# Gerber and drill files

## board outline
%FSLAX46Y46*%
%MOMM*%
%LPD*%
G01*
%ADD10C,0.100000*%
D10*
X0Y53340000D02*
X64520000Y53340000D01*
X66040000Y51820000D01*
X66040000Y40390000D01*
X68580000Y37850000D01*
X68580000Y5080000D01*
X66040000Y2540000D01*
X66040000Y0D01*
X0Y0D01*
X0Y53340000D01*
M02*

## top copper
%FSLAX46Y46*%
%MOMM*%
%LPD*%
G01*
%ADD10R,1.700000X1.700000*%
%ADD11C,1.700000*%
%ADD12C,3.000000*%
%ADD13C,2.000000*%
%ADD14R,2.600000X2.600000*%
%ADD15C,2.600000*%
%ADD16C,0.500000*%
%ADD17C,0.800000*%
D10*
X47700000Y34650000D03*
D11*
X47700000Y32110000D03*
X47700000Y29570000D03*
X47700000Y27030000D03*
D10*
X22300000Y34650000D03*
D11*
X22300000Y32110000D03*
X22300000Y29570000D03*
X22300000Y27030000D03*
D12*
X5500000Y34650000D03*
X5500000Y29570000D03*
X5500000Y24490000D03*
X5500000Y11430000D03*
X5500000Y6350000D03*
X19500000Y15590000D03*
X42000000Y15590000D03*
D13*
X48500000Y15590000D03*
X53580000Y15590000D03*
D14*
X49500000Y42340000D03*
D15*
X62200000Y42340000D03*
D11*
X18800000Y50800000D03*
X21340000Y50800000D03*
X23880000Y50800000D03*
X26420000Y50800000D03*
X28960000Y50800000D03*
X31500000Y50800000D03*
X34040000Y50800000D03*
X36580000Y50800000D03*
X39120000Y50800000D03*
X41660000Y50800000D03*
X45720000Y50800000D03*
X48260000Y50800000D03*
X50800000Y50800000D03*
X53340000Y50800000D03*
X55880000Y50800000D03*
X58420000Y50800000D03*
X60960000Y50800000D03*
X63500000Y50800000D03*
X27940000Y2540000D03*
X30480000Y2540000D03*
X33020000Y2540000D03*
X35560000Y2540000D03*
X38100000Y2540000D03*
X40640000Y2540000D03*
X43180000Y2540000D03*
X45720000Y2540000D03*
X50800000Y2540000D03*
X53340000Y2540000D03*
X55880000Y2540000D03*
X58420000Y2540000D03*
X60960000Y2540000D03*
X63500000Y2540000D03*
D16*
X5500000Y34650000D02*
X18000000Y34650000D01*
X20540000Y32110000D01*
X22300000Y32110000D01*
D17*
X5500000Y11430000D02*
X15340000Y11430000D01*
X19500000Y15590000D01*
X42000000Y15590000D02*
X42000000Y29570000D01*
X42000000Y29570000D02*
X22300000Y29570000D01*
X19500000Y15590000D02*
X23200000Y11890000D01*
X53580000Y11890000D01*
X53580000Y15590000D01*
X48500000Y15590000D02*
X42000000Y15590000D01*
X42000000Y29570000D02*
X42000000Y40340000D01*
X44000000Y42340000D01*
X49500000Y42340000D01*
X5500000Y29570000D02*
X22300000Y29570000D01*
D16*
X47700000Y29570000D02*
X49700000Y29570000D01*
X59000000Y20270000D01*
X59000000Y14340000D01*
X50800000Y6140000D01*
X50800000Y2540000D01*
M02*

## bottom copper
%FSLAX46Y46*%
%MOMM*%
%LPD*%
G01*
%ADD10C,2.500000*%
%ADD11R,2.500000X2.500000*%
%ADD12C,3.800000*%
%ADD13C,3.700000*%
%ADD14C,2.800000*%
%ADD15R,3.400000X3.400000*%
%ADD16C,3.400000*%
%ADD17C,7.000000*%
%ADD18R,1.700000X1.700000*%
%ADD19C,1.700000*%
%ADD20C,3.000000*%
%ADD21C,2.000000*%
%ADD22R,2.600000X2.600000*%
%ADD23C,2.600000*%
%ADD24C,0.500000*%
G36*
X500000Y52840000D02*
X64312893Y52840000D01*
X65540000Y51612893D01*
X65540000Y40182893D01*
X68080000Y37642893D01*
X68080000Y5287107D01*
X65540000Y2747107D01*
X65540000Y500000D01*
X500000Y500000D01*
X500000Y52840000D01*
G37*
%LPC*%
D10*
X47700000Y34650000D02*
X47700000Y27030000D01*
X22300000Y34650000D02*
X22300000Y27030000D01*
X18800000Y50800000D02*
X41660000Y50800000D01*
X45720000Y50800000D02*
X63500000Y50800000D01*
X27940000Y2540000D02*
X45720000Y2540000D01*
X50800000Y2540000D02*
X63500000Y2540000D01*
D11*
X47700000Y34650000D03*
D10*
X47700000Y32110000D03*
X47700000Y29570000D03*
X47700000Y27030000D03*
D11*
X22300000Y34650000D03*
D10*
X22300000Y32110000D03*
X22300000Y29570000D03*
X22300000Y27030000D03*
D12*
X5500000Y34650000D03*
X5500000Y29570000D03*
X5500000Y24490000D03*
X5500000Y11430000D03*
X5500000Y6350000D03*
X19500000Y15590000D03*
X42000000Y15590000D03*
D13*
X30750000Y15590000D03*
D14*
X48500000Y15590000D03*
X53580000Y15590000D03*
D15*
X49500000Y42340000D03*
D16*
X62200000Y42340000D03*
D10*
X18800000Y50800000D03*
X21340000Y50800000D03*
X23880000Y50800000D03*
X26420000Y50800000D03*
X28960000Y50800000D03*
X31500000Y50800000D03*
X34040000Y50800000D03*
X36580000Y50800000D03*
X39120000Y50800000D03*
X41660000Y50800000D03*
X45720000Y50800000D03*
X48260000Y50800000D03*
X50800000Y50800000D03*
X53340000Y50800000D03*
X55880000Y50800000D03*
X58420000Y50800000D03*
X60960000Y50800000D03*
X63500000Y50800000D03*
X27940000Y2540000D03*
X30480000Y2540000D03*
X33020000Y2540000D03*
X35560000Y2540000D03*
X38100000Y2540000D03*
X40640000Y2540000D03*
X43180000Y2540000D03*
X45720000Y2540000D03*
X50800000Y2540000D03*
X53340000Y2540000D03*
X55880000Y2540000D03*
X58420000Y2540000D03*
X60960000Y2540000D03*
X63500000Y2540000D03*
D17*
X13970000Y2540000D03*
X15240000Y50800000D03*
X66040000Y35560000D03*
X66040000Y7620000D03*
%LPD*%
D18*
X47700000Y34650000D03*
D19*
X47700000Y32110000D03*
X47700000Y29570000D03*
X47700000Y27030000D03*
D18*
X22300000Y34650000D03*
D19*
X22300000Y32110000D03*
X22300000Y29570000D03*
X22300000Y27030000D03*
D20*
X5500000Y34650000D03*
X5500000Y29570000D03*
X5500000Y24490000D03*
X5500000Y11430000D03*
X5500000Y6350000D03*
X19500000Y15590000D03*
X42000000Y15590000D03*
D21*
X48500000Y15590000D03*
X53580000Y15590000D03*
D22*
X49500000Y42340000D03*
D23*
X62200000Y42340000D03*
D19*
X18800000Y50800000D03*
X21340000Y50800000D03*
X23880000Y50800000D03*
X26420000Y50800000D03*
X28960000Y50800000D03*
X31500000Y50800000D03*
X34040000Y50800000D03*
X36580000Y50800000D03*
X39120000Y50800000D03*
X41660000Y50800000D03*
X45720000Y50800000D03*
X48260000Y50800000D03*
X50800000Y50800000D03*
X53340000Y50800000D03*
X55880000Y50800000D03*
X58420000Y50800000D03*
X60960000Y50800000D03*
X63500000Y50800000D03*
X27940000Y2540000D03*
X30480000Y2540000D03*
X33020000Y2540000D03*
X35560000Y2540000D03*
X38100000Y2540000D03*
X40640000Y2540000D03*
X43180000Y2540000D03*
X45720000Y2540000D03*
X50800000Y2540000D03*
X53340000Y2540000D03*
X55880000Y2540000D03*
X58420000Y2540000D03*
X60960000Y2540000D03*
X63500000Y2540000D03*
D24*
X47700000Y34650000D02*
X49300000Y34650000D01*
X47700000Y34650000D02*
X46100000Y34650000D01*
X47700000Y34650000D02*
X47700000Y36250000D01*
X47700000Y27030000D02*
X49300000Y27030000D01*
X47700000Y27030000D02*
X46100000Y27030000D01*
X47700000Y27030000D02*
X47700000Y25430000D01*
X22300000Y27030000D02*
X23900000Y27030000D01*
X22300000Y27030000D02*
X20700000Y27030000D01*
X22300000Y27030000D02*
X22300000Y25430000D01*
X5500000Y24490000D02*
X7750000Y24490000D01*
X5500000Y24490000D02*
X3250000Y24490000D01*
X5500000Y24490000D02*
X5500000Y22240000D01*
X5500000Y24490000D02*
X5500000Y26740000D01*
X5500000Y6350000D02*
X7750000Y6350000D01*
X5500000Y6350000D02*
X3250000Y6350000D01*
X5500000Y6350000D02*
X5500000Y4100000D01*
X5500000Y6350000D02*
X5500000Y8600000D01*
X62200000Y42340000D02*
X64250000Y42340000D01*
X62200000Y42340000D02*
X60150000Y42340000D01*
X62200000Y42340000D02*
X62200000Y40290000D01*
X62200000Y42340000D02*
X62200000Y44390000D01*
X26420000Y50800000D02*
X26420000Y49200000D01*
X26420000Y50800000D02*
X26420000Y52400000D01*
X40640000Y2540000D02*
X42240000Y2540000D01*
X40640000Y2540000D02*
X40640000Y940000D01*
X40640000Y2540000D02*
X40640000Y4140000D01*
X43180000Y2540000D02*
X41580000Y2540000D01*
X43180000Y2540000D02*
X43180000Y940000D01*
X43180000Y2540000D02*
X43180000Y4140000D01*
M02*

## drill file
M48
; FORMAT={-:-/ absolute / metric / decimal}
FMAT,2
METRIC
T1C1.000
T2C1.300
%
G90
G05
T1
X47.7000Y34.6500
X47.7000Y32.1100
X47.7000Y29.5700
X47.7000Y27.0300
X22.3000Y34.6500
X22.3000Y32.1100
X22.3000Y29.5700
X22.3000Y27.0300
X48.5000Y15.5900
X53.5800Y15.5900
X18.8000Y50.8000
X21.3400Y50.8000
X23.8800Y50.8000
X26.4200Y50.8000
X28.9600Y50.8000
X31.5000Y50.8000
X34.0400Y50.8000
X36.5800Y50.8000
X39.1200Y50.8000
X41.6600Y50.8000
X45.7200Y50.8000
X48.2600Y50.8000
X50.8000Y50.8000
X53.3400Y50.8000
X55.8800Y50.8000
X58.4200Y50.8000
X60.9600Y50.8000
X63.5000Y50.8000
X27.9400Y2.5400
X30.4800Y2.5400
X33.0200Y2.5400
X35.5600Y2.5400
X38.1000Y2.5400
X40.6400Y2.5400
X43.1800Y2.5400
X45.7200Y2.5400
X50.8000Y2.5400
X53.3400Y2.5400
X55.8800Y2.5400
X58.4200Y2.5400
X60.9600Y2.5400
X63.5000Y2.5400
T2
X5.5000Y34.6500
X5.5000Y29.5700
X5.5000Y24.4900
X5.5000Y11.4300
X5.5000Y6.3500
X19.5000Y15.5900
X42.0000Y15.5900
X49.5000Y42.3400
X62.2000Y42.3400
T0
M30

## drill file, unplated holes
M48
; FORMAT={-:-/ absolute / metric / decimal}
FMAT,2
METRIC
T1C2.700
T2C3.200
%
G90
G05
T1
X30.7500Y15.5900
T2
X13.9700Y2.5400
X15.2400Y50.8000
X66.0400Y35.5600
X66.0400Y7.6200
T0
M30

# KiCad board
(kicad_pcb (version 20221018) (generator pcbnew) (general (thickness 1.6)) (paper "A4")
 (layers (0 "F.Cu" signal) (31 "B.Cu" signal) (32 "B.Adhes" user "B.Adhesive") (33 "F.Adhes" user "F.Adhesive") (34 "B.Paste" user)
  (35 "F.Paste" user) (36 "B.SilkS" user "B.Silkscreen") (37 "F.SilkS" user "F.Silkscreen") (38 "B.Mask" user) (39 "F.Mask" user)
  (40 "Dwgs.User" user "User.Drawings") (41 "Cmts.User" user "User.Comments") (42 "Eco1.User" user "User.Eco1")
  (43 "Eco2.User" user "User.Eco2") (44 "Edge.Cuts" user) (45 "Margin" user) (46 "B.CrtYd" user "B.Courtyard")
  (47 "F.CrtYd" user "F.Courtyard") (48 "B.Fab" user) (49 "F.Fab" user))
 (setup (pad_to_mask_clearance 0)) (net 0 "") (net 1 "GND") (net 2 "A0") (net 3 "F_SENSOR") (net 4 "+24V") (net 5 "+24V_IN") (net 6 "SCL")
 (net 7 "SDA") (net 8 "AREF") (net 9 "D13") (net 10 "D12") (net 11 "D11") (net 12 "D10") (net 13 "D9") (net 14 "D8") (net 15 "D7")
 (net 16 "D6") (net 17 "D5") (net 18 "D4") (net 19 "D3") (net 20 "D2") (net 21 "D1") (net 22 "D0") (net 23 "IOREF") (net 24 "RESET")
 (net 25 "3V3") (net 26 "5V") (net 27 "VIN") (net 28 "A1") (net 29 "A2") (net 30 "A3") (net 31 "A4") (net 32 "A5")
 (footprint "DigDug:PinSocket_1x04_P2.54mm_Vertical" (layer "F.Cu") (at 147.7 118.69)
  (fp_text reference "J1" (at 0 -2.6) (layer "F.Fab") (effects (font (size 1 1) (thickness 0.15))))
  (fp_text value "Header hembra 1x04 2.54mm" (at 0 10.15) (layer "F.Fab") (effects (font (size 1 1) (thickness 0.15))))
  (pad "1" thru_hole rect (at 0 0) (size 1.7 1.7) (drill 1) (layers "*.Cu" "*.Mask") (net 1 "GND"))
  (pad "2" thru_hole circle (at 0 2.54) (size 1.7 1.7) (drill 1) (layers "*.Cu" "*.Mask"))
  (pad "3" thru_hole circle (at 0 5.08) (size 1.7 1.7) (drill 1) (layers "*.Cu" "*.Mask") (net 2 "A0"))
  (pad "4" thru_hole circle (at 0 7.62) (size 1.7 1.7) (drill 1) (layers "*.Cu" "*.Mask") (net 1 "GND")))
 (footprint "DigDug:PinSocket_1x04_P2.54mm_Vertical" (layer "F.Cu") (at 122.3 118.69)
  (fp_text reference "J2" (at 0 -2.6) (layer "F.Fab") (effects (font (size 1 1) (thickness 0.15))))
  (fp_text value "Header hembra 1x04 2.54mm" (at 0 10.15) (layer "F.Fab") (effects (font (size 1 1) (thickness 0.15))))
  (pad "1" thru_hole rect (at 0 0) (size 1.7 1.7) (drill 1) (layers "*.Cu" "*.Mask"))
  (pad "2" thru_hole circle (at 0 2.54) (size 1.7 1.7) (drill 1) (layers "*.Cu" "*.Mask") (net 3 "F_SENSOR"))
  (pad "3" thru_hole circle (at 0 5.08) (size 1.7 1.7) (drill 1) (layers "*.Cu" "*.Mask") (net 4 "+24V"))
  (pad "4" thru_hole circle (at 0 7.62) (size 1.7 1.7) (drill 1) (layers "*.Cu" "*.Mask") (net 1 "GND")))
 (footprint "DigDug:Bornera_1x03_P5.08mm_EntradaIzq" (layer "F.Cu") (at 105.5 118.69)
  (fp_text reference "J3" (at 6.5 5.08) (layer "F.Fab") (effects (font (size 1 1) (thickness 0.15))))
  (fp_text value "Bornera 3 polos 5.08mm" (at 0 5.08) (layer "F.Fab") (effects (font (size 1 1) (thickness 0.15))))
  (pad "1" thru_hole circle (at 0 0) (size 3 3) (drill 1.3) (layers "*.Cu" "*.Mask") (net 3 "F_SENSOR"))
  (pad "2" thru_hole circle (at 0 5.08) (size 3 3) (drill 1.3) (layers "*.Cu" "*.Mask") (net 4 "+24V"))
  (pad "3" thru_hole circle (at 0 10.16) (size 3 3) (drill 1.3) (layers "*.Cu" "*.Mask") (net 1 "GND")))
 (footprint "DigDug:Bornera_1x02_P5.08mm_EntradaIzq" (layer "F.Cu") (at 105.5 141.91)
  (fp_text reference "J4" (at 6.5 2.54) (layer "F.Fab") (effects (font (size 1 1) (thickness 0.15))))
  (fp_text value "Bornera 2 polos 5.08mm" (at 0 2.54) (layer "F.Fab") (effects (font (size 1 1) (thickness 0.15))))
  (pad "1" thru_hole circle (at 0 0) (size 3 3) (drill 1.3) (layers "*.Cu" "*.Mask") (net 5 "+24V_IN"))
  (pad "2" thru_hole circle (at 0 5.08) (size 3 3) (drill 1.3) (layers "*.Cu" "*.Mask") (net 1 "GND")))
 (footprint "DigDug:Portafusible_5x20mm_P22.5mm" (layer "F.Cu") (at 119.5 137.75)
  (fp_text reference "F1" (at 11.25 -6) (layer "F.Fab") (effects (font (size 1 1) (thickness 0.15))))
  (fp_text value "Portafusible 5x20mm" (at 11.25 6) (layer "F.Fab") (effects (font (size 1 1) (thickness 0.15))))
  (pad "1" thru_hole circle (at 0 0) (size 3 3) (drill 1.3) (layers "*.Cu" "*.Mask") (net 5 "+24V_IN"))
  (pad "2" thru_hole circle (at 22.5 0) (size 3 3) (drill 1.3) (layers "*.Cu" "*.Mask") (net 4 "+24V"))
  (pad "" np_thru_hole circle (at 11.25 0) (size 2.7 2.7) (drill 2.7) (layers "*.Cu" "*.Mask")))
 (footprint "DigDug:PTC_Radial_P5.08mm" (layer "F.Cu") (at 148.5 137.75)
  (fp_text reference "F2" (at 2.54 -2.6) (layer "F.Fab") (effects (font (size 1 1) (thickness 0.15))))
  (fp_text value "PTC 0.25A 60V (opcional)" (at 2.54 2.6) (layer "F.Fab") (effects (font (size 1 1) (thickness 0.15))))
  (pad "1" thru_hole circle (at 0 0) (size 2 2) (drill 1) (layers "*.Cu" "*.Mask") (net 4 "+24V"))
  (pad "2" thru_hole circle (at 5.08 0) (size 2 2) (drill 1) (layers "*.Cu" "*.Mask") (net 5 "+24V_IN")))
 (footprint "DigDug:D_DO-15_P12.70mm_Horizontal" (layer "F.Cu") (at 149.5 111)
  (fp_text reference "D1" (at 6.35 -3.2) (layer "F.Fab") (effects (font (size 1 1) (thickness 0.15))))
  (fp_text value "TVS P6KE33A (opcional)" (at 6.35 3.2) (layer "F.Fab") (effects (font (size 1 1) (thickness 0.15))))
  (pad "1" thru_hole rect (at 0 0) (size 2.6 2.6) (drill 1.3) (layers "*.Cu" "*.Mask") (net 4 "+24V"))
  (pad "2" thru_hole circle (at 12.7 0) (size 2.6 2.6) (drill 1.3) (layers "*.Cu" "*.Mask") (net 1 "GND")))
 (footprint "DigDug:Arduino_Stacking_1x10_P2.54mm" (layer "F.Cu") (at 118.8 102.54)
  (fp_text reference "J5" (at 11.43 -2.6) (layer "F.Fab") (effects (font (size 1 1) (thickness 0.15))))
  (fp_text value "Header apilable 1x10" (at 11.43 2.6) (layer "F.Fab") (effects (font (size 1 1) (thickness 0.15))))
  (pad "1" thru_hole circle (at 0 0) (size 1.7 1.7) (drill 1) (layers "*.Cu" "*.Mask") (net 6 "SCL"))
  (pad "2" thru_hole circle (at 2.54 0) (size 1.7 1.7) (drill 1) (layers "*.Cu" "*.Mask") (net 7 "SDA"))
  (pad "3" thru_hole circle (at 5.08 0) (size 1.7 1.7) (drill 1) (layers "*.Cu" "*.Mask") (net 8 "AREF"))
  (pad "4" thru_hole circle (at 7.62 0) (size 1.7 1.7) (drill 1) (layers "*.Cu" "*.Mask") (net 1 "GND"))
  (pad "5" thru_hole circle (at 10.16 0) (size 1.7 1.7) (drill 1) (layers "*.Cu" "*.Mask") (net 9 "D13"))
  (pad "6" thru_hole circle (at 12.7 0) (size 1.7 1.7) (drill 1) (layers "*.Cu" "*.Mask") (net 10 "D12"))
  (pad "7" thru_hole circle (at 15.24 0) (size 1.7 1.7) (drill 1) (layers "*.Cu" "*.Mask") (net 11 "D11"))
  (pad "8" thru_hole circle (at 17.78 0) (size 1.7 1.7) (drill 1) (layers "*.Cu" "*.Mask") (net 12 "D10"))
  (pad "9" thru_hole circle (at 20.32 0) (size 1.7 1.7) (drill 1) (layers "*.Cu" "*.Mask") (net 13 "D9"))
  (pad "10" thru_hole circle (at 22.86 0) (size 1.7 1.7) (drill 1) (layers "*.Cu" "*.Mask") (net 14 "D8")))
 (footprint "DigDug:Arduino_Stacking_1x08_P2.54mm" (layer "F.Cu") (at 145.72 102.54)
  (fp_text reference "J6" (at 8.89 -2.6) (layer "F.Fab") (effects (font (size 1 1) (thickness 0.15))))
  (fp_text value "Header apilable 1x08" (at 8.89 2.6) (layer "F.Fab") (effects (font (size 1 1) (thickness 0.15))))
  (pad "1" thru_hole circle (at 0 0) (size 1.7 1.7) (drill 1) (layers "*.Cu" "*.Mask") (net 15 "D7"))
  (pad "2" thru_hole circle (at 2.54 0) (size 1.7 1.7) (drill 1) (layers "*.Cu" "*.Mask") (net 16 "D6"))
  (pad "3" thru_hole circle (at 5.08 0) (size 1.7 1.7) (drill 1) (layers "*.Cu" "*.Mask") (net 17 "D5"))
  (pad "4" thru_hole circle (at 7.62 0) (size 1.7 1.7) (drill 1) (layers "*.Cu" "*.Mask") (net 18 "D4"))
  (pad "5" thru_hole circle (at 10.16 0) (size 1.7 1.7) (drill 1) (layers "*.Cu" "*.Mask") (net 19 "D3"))
  (pad "6" thru_hole circle (at 12.7 0) (size 1.7 1.7) (drill 1) (layers "*.Cu" "*.Mask") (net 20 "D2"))
  (pad "7" thru_hole circle (at 15.24 0) (size 1.7 1.7) (drill 1) (layers "*.Cu" "*.Mask") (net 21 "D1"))
  (pad "8" thru_hole circle (at 17.78 0) (size 1.7 1.7) (drill 1) (layers "*.Cu" "*.Mask") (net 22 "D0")))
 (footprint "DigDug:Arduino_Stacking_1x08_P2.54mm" (layer "F.Cu") (at 127.94 150.8)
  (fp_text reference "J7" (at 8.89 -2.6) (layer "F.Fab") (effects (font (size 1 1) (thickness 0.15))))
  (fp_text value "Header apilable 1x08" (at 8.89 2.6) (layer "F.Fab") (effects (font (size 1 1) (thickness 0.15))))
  (pad "1" thru_hole circle (at 0 0) (size 1.7 1.7) (drill 1) (layers "*.Cu" "*.Mask"))
  (pad "2" thru_hole circle (at 2.54 0) (size 1.7 1.7) (drill 1) (layers "*.Cu" "*.Mask") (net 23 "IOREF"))
  (pad "3" thru_hole circle (at 5.08 0) (size 1.7 1.7) (drill 1) (layers "*.Cu" "*.Mask") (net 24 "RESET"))
  (pad "4" thru_hole circle (at 7.62 0) (size 1.7 1.7) (drill 1) (layers "*.Cu" "*.Mask") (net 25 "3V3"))
  (pad "5" thru_hole circle (at 10.16 0) (size 1.7 1.7) (drill 1) (layers "*.Cu" "*.Mask") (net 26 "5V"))
  (pad "6" thru_hole circle (at 12.7 0) (size 1.7 1.7) (drill 1) (layers "*.Cu" "*.Mask") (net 1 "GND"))
  (pad "7" thru_hole circle (at 15.24 0) (size 1.7 1.7) (drill 1) (layers "*.Cu" "*.Mask") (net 1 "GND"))
  (pad "8" thru_hole circle (at 17.78 0) (size 1.7 1.7) (drill 1) (layers "*.Cu" "*.Mask") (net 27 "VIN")))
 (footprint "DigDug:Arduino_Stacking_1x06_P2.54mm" (layer "F.Cu") (at 150.8 150.8)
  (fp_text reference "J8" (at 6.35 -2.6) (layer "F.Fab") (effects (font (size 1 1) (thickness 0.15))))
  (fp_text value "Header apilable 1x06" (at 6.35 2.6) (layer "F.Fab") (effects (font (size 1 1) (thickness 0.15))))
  (pad "1" thru_hole circle (at 0 0) (size 1.7 1.7) (drill 1) (layers "*.Cu" "*.Mask") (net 2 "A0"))
  (pad "2" thru_hole circle (at 2.54 0) (size 1.7 1.7) (drill 1) (layers "*.Cu" "*.Mask") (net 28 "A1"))
  (pad "3" thru_hole circle (at 5.08 0) (size 1.7 1.7) (drill 1) (layers "*.Cu" "*.Mask") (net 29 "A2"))
  (pad "4" thru_hole circle (at 7.62 0) (size 1.7 1.7) (drill 1) (layers "*.Cu" "*.Mask") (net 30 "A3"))
  (pad "5" thru_hole circle (at 10.16 0) (size 1.7 1.7) (drill 1) (layers "*.Cu" "*.Mask") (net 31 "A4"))
  (pad "6" thru_hole circle (at 12.7 0) (size 1.7 1.7) (drill 1) (layers "*.Cu" "*.Mask") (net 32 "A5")))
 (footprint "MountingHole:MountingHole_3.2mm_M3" (layer "F.Cu") (at 113.97 150.8)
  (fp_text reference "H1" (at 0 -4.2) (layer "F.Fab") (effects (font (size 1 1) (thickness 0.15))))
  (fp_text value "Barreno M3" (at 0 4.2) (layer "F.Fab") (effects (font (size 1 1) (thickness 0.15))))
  (pad "" np_thru_hole circle (at 0 0) (size 3.2 3.2) (drill 3.2) (layers "*.Cu" "*.Mask")))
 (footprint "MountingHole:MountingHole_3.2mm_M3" (layer "F.Cu") (at 115.24 102.54)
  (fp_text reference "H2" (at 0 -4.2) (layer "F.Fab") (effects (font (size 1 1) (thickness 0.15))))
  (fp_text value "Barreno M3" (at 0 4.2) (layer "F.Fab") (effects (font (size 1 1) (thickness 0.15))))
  (pad "" np_thru_hole circle (at 0 0) (size 3.2 3.2) (drill 3.2) (layers "*.Cu" "*.Mask")))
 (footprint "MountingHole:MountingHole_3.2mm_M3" (layer "F.Cu") (at 166.04 117.78)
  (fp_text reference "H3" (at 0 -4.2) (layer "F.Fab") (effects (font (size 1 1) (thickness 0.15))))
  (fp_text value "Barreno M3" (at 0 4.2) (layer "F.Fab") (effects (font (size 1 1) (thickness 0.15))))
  (pad "" np_thru_hole circle (at 0 0) (size 3.2 3.2) (drill 3.2) (layers "*.Cu" "*.Mask")))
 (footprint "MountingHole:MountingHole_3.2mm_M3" (layer "F.Cu") (at 166.04 145.72)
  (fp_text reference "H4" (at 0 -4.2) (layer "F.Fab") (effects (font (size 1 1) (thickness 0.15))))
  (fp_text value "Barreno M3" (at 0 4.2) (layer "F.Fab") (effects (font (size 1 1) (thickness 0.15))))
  (pad "" np_thru_hole circle (at 0 0) (size 3.2 3.2) (drill 3.2) (layers "*.Cu" "*.Mask")))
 (gr_line (start 100 100) (end 164.52 100) (stroke (width 0.1) (type default)) (layer "Edge.Cuts"))
 (gr_line (start 164.52 100) (end 166.04 101.52) (stroke (width 0.1) (type default)) (layer "Edge.Cuts"))
 (gr_line (start 166.04 101.52) (end 166.04 112.95) (stroke (width 0.1) (type default)) (layer "Edge.Cuts"))
 (gr_line (start 166.04 112.95) (end 168.58 115.49) (stroke (width 0.1) (type default)) (layer "Edge.Cuts"))
 (gr_line (start 168.58 115.49) (end 168.58 148.26) (stroke (width 0.1) (type default)) (layer "Edge.Cuts"))
 (gr_line (start 168.58 148.26) (end 166.04 150.8) (stroke (width 0.1) (type default)) (layer "Edge.Cuts"))
 (gr_line (start 166.04 150.8) (end 166.04 153.34) (stroke (width 0.1) (type default)) (layer "Edge.Cuts"))
 (gr_line (start 166.04 153.34) (end 100 153.34) (stroke (width 0.1) (type default)) (layer "Edge.Cuts"))
 (gr_line (start 100 153.34) (end 100 100) (stroke (width 0.1) (type default)) (layer "Edge.Cuts"))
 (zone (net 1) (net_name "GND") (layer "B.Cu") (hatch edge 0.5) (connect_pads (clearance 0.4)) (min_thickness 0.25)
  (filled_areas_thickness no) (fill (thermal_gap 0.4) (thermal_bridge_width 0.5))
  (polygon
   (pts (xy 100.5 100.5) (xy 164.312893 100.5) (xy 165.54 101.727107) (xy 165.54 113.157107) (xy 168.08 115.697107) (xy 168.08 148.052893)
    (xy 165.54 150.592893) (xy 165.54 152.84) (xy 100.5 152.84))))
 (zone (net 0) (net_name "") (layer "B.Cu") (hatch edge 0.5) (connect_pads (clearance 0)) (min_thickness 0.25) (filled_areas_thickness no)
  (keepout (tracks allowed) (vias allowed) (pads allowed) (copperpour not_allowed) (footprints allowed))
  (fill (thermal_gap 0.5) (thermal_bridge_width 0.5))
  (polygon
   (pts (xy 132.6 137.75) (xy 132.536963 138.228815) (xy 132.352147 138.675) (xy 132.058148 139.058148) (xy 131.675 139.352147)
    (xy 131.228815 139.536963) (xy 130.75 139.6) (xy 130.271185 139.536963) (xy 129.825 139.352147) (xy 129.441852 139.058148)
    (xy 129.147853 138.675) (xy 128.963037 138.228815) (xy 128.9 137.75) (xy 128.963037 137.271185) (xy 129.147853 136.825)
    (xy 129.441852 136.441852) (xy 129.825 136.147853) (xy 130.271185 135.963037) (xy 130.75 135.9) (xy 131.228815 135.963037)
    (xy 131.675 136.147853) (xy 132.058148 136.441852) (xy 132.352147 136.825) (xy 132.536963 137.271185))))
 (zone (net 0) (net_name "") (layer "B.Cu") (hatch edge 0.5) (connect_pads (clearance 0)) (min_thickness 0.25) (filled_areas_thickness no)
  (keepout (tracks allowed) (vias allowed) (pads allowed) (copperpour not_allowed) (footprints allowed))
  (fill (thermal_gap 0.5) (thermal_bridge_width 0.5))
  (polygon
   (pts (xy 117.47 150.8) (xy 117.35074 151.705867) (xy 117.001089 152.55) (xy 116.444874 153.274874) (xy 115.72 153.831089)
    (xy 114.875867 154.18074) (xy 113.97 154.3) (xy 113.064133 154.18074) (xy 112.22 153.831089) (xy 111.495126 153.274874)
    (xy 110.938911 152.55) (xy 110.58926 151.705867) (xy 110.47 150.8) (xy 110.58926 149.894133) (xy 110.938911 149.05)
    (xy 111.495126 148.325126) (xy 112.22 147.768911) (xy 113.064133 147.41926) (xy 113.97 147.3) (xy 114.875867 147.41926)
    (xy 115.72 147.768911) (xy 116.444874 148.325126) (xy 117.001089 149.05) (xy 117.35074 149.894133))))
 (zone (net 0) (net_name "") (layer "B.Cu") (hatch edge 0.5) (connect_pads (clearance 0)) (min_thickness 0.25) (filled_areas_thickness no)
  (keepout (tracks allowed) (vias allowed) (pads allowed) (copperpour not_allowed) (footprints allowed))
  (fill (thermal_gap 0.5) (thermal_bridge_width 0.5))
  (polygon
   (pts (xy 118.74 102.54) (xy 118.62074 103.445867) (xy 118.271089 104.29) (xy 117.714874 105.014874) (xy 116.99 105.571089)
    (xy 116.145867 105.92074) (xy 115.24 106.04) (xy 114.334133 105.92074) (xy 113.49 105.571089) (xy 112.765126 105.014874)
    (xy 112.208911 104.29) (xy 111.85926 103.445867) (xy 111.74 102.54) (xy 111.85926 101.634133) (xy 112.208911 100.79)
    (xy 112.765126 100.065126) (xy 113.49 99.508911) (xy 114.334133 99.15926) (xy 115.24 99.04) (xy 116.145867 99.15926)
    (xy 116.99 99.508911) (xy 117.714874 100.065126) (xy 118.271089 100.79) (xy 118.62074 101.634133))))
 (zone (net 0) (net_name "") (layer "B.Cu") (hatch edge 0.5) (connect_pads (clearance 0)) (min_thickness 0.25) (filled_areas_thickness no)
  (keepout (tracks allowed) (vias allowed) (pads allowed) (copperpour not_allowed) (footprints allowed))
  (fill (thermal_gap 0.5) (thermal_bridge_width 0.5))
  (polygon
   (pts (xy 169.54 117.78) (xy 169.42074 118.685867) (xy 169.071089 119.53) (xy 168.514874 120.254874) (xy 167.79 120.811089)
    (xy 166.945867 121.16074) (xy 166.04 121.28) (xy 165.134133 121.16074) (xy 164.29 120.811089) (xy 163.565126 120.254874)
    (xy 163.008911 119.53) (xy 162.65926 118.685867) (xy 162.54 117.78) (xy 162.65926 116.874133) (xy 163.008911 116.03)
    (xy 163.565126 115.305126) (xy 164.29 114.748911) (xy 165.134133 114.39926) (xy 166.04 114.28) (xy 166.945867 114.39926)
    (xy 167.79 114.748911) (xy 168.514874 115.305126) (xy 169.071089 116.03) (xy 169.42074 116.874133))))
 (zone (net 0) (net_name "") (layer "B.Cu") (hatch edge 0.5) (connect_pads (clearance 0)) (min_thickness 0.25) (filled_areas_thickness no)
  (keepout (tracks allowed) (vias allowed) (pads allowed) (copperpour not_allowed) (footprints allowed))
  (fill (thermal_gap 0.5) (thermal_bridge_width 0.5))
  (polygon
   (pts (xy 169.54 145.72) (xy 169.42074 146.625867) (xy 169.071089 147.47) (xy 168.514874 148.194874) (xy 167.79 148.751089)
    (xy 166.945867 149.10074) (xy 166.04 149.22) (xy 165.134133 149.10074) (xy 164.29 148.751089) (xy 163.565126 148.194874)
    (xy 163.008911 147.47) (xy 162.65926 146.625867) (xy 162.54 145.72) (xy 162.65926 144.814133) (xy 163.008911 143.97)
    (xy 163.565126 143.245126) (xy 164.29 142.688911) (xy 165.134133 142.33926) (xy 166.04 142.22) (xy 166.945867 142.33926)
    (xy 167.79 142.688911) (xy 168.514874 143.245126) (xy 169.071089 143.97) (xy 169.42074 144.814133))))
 (segment (start 105.5 118.69) (end 118 118.69) (width 0.5) (layer "F.Cu") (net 3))
 (segment (start 118 118.69) (end 120.54 121.23) (width 0.5) (layer "F.Cu") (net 3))
 (segment (start 120.54 121.23) (end 122.3 121.23) (width 0.5) (layer "F.Cu") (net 3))
 (segment (start 105.5 141.91) (end 115.34 141.91) (width 0.8) (layer "F.Cu") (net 5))
 (segment (start 115.34 141.91) (end 119.5 137.75) (width 0.8) (layer "F.Cu") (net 5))
 (segment (start 142 137.75) (end 142 123.77) (width 0.8) (layer "F.Cu") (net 4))
 (segment (start 142 123.77) (end 122.3 123.77) (width 0.8) (layer "F.Cu") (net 4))
 (segment (start 119.5 137.75) (end 123.2 141.45) (width 0.8) (layer "F.Cu") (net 5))
 (segment (start 123.2 141.45) (end 153.58 141.45) (width 0.8) (layer "F.Cu") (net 5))
 (segment (start 153.58 141.45) (end 153.58 137.75) (width 0.8) (layer "F.Cu") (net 5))
 (segment (start 148.5 137.75) (end 142 137.75) (width 0.8) (layer "F.Cu") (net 4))
 (segment (start 142 123.77) (end 142 113) (width 0.8) (layer "F.Cu") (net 4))
 (segment (start 142 113) (end 144 111) (width 0.8) (layer "F.Cu") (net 4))
 (segment (start 144 111) (end 149.5 111) (width 0.8) (layer "F.Cu") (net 4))
 (segment (start 105.5 123.77) (end 122.3 123.77) (width 0.8) (layer "F.Cu") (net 4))
 (segment (start 147.7 123.77) (end 149.7 123.77) (width 0.5) (layer "F.Cu") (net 2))
 (segment (start 149.7 123.77) (end 159 133.07) (width 0.5) (layer "F.Cu") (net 2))
 (segment (start 159 133.07) (end 159 139) (width 0.5) (layer "F.Cu") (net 2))
 (segment (start 159 139) (end 150.8 147.2) (width 0.5) (layer "F.Cu") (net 2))
 (segment (start 150.8 147.2) (end 150.8 150.8) (width 0.5) (layer "F.Cu") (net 2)))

